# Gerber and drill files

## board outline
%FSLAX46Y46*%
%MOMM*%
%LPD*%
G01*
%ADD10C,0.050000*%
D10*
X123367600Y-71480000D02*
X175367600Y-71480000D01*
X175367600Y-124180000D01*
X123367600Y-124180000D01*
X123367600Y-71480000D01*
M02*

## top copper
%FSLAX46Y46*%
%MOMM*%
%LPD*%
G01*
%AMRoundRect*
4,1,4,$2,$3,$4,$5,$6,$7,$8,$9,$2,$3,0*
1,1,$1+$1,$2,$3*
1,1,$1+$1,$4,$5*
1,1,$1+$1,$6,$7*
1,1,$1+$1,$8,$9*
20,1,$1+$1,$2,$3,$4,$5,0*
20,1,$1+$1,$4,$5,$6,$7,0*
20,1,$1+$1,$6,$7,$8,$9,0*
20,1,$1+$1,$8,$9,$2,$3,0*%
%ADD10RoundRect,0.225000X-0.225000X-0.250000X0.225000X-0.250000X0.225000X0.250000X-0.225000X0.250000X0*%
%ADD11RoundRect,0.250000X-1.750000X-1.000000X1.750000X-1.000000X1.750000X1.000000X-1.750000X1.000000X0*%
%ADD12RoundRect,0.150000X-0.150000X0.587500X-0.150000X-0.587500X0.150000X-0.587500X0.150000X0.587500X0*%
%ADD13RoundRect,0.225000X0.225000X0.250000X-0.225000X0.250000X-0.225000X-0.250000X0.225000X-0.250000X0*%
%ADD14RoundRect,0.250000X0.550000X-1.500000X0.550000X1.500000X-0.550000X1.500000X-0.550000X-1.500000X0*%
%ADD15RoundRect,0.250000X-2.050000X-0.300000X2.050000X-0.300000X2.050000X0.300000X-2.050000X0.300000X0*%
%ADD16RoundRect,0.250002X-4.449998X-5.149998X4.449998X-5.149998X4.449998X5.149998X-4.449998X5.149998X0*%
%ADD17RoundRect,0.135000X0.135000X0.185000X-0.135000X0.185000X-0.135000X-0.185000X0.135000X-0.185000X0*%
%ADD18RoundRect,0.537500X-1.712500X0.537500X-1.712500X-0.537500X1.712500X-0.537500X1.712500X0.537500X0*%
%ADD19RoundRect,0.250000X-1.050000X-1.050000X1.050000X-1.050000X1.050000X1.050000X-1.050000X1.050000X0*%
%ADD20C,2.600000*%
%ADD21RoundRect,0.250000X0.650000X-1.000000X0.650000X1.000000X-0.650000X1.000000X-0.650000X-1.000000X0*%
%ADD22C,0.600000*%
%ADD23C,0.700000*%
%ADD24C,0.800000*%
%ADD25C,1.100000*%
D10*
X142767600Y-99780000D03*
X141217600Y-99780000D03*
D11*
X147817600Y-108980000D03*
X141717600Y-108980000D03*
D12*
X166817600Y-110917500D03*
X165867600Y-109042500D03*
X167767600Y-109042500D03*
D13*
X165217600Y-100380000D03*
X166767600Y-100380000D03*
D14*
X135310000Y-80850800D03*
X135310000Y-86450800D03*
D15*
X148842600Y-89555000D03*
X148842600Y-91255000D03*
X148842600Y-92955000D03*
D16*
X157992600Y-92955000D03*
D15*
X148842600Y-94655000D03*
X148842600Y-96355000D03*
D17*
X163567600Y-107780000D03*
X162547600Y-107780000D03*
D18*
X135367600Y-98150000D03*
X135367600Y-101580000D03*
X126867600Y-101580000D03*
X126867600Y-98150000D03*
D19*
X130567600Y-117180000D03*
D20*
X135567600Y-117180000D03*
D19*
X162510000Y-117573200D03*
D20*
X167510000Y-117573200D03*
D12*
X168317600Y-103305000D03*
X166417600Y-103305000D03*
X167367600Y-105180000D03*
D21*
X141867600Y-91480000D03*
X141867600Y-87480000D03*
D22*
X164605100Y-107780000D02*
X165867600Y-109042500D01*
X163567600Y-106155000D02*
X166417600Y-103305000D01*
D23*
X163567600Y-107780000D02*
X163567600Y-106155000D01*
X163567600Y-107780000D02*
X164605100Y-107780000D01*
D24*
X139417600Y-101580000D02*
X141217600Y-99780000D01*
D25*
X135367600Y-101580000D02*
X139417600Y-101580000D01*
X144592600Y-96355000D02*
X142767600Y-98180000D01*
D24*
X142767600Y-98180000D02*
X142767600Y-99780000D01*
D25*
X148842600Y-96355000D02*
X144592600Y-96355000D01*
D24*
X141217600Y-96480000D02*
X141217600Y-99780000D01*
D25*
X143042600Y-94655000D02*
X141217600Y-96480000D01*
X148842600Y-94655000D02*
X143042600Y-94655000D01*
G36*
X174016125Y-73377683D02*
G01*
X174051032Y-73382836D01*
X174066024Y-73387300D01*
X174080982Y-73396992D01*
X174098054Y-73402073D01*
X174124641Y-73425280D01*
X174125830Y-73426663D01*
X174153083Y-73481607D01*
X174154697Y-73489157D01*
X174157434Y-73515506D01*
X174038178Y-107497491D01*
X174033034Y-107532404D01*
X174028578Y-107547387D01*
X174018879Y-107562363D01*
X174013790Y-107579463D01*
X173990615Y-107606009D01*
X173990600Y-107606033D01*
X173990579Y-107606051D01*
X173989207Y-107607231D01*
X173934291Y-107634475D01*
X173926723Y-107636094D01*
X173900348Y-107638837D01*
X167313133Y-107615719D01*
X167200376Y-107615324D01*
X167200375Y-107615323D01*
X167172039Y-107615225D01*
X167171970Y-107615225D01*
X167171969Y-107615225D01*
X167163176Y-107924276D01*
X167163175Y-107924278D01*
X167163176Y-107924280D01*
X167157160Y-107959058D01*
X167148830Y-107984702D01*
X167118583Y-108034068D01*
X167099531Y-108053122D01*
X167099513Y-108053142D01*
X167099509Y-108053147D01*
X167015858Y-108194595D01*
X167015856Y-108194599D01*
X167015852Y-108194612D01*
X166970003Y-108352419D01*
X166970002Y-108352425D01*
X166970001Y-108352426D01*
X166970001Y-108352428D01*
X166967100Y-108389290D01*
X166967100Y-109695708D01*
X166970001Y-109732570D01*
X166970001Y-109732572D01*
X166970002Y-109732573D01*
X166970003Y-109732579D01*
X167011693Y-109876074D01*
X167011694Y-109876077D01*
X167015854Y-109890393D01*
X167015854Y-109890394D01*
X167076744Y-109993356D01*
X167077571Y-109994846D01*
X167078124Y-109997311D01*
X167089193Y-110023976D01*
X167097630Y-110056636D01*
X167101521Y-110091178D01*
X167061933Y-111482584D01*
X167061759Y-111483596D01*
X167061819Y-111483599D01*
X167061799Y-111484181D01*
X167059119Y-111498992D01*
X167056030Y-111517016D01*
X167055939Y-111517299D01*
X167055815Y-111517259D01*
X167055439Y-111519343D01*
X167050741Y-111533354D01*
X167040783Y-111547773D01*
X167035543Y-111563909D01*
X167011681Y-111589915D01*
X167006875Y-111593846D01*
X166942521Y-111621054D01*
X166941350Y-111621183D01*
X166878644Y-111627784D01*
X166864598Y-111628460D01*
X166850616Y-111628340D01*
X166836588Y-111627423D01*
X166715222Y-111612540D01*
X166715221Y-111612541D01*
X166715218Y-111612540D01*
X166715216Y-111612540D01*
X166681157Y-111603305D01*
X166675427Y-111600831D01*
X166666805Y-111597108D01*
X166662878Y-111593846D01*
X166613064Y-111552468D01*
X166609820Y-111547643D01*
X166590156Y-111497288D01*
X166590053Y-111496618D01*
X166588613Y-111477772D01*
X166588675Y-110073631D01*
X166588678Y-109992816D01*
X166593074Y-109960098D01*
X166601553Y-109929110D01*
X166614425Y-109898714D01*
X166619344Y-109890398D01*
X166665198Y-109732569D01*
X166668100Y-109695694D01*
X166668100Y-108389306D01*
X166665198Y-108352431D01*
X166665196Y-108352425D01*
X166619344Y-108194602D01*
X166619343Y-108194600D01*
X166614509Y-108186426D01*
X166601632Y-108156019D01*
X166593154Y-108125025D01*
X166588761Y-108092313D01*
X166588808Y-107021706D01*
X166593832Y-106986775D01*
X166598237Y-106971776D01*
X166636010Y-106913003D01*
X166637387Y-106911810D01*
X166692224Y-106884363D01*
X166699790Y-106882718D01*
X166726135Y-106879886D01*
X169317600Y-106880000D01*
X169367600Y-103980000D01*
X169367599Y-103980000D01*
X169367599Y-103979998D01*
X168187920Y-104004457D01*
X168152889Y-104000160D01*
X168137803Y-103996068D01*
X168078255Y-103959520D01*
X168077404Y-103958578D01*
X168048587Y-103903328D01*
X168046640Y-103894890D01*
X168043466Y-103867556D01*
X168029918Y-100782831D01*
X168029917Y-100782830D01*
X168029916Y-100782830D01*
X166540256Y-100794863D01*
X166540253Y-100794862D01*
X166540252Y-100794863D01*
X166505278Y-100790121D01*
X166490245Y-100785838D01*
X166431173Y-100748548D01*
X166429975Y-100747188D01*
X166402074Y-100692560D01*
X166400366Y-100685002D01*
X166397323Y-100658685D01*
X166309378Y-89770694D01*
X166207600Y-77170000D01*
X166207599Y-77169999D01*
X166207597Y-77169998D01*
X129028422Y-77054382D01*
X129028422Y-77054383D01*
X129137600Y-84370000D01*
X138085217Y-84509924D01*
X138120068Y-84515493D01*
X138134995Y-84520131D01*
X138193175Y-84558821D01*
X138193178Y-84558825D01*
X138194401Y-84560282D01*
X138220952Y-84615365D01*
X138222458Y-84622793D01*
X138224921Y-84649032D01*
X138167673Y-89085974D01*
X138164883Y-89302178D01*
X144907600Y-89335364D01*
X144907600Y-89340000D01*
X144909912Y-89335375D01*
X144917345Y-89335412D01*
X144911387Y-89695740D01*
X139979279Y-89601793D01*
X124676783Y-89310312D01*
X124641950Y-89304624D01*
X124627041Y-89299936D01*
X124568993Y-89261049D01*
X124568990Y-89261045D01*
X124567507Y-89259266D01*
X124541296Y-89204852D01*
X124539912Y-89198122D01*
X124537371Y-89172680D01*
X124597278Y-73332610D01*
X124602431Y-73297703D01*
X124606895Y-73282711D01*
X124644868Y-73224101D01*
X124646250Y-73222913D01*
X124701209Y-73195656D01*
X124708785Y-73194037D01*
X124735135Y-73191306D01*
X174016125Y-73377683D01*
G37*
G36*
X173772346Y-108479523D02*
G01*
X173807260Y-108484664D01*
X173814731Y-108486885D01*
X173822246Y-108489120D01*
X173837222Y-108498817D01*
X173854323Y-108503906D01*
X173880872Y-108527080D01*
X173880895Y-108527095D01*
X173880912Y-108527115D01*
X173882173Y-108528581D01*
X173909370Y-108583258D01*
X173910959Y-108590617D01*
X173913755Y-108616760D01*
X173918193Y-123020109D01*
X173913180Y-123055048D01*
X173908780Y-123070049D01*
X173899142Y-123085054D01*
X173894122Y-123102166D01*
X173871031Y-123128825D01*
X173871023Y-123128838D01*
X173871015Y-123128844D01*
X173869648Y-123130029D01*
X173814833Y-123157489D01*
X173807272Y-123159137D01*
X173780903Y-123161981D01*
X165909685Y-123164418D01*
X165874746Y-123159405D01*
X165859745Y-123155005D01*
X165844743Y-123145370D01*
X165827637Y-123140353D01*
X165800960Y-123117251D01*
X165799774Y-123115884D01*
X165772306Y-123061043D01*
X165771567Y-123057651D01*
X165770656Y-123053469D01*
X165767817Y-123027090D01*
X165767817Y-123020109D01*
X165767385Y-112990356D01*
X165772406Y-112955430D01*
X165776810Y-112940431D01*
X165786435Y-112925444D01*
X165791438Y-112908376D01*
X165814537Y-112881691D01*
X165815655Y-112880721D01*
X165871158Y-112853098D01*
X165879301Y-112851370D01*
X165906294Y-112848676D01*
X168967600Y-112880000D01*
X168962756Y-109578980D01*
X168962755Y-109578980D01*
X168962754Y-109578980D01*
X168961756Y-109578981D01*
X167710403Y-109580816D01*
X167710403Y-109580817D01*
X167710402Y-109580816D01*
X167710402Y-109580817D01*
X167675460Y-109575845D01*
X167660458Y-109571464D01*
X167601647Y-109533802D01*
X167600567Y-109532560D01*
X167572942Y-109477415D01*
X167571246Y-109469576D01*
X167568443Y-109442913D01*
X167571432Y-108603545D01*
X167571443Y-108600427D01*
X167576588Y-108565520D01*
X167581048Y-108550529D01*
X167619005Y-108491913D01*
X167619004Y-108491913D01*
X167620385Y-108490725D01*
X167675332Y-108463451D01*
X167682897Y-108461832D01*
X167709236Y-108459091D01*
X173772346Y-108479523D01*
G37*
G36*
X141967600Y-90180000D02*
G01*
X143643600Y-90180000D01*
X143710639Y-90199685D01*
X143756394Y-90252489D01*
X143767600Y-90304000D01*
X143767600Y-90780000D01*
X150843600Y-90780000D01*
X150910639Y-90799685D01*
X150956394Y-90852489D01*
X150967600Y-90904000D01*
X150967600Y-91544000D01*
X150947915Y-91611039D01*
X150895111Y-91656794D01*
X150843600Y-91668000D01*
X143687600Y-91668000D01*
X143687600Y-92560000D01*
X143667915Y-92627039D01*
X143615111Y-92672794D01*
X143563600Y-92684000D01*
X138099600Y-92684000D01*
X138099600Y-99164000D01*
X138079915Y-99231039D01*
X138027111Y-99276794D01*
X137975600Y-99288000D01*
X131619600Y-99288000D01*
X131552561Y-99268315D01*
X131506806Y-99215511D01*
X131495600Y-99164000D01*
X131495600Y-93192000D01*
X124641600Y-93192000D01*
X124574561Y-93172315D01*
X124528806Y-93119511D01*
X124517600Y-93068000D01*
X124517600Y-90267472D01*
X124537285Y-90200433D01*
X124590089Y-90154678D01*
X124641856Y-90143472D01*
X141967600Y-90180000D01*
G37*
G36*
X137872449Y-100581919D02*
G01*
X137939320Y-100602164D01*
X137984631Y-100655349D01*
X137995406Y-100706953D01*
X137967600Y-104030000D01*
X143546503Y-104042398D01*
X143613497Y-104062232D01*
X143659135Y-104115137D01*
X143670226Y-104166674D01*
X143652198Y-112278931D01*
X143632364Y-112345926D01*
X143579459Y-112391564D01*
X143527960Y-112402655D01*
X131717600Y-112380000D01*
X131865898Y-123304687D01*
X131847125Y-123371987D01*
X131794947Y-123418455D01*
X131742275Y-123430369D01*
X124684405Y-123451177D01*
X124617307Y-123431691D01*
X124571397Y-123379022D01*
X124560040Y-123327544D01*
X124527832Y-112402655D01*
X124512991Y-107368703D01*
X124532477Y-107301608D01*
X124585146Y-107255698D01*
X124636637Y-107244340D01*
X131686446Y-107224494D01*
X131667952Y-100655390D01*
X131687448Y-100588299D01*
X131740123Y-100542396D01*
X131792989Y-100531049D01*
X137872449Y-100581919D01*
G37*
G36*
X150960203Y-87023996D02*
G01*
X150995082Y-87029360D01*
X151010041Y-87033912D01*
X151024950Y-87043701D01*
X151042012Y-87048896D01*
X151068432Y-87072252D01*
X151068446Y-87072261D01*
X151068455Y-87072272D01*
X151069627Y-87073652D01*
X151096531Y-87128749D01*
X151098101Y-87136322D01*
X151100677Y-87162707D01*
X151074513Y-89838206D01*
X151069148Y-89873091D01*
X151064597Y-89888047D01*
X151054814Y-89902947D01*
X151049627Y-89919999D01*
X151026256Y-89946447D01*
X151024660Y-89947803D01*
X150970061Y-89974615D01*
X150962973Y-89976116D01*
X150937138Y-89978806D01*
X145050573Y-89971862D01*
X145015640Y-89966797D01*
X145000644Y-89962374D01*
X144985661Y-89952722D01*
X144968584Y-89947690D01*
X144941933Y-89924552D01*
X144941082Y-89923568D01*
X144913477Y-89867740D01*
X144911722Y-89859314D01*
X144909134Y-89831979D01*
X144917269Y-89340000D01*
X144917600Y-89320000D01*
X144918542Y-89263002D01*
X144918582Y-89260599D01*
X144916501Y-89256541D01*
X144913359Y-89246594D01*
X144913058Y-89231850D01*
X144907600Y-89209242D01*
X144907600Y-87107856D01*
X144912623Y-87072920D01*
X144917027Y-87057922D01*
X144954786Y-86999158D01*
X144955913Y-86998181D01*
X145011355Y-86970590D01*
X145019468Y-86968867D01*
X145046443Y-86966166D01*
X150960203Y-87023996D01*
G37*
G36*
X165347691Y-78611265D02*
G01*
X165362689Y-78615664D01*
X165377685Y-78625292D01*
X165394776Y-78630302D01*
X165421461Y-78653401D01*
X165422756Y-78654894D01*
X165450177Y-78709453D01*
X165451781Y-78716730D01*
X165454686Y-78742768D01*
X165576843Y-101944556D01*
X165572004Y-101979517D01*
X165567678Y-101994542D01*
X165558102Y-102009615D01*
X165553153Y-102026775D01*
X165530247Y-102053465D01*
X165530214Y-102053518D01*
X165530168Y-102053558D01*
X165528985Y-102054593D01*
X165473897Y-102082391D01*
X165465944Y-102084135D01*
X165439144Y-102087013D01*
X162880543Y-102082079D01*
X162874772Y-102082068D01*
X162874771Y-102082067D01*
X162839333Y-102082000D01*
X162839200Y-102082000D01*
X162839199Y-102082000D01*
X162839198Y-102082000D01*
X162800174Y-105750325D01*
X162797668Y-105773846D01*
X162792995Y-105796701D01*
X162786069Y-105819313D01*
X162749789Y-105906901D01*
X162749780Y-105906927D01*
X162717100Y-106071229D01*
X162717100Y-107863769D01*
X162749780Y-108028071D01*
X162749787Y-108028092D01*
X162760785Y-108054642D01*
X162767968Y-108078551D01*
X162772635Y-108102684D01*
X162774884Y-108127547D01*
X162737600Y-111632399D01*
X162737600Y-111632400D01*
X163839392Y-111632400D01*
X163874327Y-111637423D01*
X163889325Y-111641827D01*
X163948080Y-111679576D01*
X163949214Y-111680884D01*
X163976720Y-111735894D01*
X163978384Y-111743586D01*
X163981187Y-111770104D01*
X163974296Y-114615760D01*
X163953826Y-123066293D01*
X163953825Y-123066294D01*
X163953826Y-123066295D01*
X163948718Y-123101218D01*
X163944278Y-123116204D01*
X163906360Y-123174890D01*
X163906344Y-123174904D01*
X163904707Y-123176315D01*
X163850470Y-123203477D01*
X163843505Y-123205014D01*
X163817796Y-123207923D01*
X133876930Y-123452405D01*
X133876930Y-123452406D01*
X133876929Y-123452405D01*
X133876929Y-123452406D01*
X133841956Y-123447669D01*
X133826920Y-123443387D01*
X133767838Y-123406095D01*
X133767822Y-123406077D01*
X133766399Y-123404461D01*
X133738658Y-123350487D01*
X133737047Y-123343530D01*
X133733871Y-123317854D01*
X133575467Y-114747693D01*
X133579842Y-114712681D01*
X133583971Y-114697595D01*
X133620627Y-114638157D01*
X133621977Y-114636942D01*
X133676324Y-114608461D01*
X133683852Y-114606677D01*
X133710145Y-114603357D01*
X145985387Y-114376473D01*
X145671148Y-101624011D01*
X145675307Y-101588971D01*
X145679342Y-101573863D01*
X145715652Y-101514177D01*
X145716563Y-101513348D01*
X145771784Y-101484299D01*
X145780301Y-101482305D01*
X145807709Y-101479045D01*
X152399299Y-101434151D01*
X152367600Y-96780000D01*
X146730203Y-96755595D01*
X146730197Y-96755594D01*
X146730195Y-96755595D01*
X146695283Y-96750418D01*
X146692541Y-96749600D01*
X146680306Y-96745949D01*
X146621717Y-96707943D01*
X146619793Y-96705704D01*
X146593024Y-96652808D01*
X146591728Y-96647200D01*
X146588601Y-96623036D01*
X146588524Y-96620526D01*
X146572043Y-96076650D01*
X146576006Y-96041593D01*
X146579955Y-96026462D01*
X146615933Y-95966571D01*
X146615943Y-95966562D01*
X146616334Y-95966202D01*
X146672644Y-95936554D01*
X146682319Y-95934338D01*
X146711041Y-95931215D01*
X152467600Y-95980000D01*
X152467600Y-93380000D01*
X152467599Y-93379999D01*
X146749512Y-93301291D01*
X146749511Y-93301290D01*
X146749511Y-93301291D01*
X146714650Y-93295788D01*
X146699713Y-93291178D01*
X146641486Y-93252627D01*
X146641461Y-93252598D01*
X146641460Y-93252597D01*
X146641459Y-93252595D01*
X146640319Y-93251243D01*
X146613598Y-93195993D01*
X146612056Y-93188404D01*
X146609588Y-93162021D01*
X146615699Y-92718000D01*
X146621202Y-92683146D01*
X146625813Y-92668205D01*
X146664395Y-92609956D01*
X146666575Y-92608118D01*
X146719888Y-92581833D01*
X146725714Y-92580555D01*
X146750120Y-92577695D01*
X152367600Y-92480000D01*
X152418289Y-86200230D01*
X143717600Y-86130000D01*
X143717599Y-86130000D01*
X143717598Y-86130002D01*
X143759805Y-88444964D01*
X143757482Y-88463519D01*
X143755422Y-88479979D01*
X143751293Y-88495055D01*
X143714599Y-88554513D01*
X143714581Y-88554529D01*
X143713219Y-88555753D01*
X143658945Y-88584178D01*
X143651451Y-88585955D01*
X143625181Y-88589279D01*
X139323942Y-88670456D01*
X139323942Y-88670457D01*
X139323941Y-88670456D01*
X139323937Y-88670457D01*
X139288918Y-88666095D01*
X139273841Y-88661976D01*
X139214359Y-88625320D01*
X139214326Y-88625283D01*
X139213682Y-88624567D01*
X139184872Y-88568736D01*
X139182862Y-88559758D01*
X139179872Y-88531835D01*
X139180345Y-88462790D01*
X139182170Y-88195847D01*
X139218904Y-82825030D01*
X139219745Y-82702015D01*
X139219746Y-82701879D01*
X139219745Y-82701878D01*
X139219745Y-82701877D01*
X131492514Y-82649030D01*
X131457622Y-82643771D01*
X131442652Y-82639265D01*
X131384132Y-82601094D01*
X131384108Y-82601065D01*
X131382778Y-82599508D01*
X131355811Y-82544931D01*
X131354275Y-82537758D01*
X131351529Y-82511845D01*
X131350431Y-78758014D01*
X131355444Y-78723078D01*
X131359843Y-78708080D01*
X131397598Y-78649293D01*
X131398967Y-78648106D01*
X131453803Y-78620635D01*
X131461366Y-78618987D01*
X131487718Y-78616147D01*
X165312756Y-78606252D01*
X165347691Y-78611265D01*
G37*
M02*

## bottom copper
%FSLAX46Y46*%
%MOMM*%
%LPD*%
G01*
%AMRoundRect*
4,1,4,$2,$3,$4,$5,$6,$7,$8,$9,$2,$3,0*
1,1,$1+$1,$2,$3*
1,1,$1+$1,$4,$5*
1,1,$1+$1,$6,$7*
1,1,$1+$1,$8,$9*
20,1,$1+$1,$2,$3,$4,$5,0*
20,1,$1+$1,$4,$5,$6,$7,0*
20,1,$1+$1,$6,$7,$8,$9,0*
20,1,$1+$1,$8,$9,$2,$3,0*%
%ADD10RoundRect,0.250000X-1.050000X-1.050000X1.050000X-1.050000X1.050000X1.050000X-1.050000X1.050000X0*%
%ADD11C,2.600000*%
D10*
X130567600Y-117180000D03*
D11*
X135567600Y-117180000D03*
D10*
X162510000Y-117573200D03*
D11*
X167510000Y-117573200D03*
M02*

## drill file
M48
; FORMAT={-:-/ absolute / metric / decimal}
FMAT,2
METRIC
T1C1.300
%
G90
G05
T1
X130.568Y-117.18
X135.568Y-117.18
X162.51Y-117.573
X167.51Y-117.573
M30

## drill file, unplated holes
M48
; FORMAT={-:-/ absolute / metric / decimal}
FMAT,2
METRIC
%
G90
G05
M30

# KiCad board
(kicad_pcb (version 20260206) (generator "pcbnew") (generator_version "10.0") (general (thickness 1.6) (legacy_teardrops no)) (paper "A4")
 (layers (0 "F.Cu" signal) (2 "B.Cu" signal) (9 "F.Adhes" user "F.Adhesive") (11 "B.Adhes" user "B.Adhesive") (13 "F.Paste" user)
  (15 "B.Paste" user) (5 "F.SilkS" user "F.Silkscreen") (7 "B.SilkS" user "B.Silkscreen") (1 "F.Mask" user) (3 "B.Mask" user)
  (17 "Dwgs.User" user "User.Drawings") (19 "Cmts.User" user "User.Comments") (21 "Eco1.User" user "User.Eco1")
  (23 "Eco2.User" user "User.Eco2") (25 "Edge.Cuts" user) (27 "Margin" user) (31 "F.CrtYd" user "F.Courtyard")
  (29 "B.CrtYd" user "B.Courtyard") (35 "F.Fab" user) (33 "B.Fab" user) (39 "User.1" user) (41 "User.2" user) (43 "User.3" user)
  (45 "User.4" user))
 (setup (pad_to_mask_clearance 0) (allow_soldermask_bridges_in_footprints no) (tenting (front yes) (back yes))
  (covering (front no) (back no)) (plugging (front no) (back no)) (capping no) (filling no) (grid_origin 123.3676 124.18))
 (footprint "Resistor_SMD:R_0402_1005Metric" (layer "F.Cu") (at 163.0576 107.78 180)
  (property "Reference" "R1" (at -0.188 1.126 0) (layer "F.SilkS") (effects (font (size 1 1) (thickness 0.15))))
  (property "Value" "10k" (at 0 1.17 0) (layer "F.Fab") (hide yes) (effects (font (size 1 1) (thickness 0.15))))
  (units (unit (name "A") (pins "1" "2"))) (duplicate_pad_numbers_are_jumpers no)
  (pad "1" smd roundrect (at -0.51 0 180) (size 0.54 0.64) (layers "F.Cu" "F.Mask" "F.Paste") (roundrect_rratio 0.25) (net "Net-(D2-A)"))
  (pad "2" smd roundrect (at 0.51 0 180) (size 0.54 0.64) (layers "F.Cu" "F.Mask" "F.Paste") (roundrect_rratio 0.25) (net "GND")))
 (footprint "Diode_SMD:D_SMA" (layer "F.Cu") (at 141.8676 89.48 90)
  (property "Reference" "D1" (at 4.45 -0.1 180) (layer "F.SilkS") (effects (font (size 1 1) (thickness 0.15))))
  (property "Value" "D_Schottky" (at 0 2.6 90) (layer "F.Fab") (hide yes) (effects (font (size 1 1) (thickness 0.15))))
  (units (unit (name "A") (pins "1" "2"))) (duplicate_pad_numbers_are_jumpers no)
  (pad "1" smd roundrect (at -2 0 90) (size 2.5 1.8) (layers "F.Cu" "F.Mask" "F.Paste") (roundrect_rratio 0.1388888889) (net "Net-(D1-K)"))
  (pad "2" smd roundrect (at 2 0 90) (size 2.5 1.8) (layers "F.Cu" "F.Mask" "F.Paste") (roundrect_rratio 0.1388888889) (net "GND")))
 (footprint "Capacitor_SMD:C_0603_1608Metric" (layer "F.Cu") (at 141.9926 99.78)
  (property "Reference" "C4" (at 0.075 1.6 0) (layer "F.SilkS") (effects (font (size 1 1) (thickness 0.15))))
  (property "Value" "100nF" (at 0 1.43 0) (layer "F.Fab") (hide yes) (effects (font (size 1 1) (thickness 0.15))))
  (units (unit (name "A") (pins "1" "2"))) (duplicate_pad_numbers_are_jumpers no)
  (pad "1" smd roundrect (at -0.775 0) (size 0.9 0.95) (layers "F.Cu" "F.Mask" "F.Paste") (roundrect_rratio 0.25) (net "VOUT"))
  (pad "2" smd roundrect (at 0.775 0) (size 0.9 0.95) (layers "F.Cu" "F.Mask" "F.Paste") (roundrect_rratio 0.25) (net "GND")))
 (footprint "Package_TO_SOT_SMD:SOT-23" (layer "F.Cu") (at 167.3676 104.2425 -90)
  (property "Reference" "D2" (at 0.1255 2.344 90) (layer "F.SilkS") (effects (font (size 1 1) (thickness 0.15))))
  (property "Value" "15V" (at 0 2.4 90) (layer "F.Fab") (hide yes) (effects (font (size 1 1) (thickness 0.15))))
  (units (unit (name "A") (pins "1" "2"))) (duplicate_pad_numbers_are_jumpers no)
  (pad "1" smd roundrect (at -0.9375 -0.95 270) (size 1.475 0.6) (layers "F.Cu" "F.Mask" "F.Paste") (roundrect_rratio 0.25)
   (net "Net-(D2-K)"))
  (pad "2" smd roundrect (at -0.9375 0.95 270) (size 1.475 0.6) (layers "F.Cu" "F.Mask" "F.Paste") (roundrect_rratio 0.25)
   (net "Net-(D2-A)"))
  (pad "3" smd roundrect (at 0.9375 0 270) (size 1.475 0.6) (layers "F.Cu" "F.Mask" "F.Paste") (roundrect_rratio 0.25)))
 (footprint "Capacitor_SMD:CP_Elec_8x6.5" (layer "F.Cu") (at 144.7676 108.98)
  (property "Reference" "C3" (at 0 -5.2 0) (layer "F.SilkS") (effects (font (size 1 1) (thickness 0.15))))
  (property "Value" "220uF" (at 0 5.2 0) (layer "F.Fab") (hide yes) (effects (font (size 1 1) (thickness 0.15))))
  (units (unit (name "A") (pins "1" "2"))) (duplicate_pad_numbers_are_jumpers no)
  (pad "1" smd roundrect (at -3.05 0) (size 4 2.5) (layers "F.Cu" "F.Mask" "F.Paste") (roundrect_rratio 0.1) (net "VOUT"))
  (pad "2" smd roundrect (at 3.05 0) (size 4 2.5) (layers "F.Cu" "F.Mask" "F.Paste") (roundrect_rratio 0.1) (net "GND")))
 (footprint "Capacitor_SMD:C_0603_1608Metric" (layer "F.Cu") (at 165.9926 100.38 180)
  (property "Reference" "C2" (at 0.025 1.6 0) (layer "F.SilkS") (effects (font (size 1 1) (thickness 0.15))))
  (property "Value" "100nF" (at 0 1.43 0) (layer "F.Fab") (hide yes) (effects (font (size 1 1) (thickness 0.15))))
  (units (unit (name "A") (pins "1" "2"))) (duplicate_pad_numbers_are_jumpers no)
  (pad "1" smd roundrect (at -0.775 0 180) (size 0.9 0.95) (layers "F.Cu" "F.Mask" "F.Paste") (roundrect_rratio 0.25) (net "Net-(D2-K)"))
  (pad "2" smd roundrect (at 0.775 0 180) (size 0.9 0.95) (layers "F.Cu" "F.Mask" "F.Paste") (roundrect_rratio 0.25) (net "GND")))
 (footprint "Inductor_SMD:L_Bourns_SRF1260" (layer "F.Cu") (at 131.1176 99.865 -90)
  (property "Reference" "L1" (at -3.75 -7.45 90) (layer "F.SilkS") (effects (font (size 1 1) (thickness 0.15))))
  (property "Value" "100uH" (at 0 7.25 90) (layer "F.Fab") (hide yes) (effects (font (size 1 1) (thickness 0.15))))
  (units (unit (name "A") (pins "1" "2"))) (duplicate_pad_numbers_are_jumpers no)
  (pad "1" smd roundrect (at -1.715 -4.25 270) (size 2.15 4.5) (layers "F.Cu" "F.Mask" "F.Paste") (roundrect_rratio 0.25) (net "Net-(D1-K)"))
  (pad "2" smd roundrect (at 1.715 -4.25 270) (size 2.15 4.5) (layers "F.Cu" "F.Mask" "F.Paste") (roundrect_rratio 0.25) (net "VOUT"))
  (pad "3" smd roundrect (at 1.715 4.25 270) (size 2.15 4.5) (layers "F.Cu" "F.Mask" "F.Paste") (roundrect_rratio 0.25))
  (pad "4" smd roundrect (at -1.715 4.25 270) (size 2.15 4.5) (layers "F.Cu" "F.Mask" "F.Paste") (roundrect_rratio 0.25)))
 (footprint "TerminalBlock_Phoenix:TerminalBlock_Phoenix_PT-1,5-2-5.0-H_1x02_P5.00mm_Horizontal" (layer "F.Cu") (at 130.5676 117.18)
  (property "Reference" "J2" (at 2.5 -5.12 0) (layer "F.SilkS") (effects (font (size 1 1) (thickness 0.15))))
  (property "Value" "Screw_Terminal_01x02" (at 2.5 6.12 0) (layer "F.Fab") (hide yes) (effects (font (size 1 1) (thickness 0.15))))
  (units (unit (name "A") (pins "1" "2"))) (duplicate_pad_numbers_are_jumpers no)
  (pad "1" thru_hole roundrect (at 0 0) (size 2.6 2.6) (drill 1.3) (layers "*.Cu" "*.Mask") (remove_unused_layers no)
   (roundrect_rratio 0.096154) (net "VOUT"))
  (pad "2" thru_hole circle (at 5 0) (size 2.6 2.6) (drill 1.3) (layers "*.Cu" "*.Mask") (remove_unused_layers no) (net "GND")))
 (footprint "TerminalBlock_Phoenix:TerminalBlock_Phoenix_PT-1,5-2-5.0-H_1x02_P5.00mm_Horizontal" (layer "F.Cu") (at 162.51 117.5732)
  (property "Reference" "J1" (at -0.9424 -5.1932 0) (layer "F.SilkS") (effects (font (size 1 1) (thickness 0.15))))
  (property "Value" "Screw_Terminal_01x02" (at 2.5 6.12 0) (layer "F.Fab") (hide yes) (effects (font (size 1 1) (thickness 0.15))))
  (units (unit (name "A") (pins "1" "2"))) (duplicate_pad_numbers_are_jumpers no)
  (pad "1" thru_hole roundrect (at 0 0) (size 2.6 2.6) (drill 1.3) (layers "*.Cu" "*.Mask") (remove_unused_layers no)
   (roundrect_rratio 0.096154) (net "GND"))
  (pad "2" thru_hole circle (at 5 0) (size 2.6 2.6) (drill 1.3) (layers "*.Cu" "*.Mask") (remove_unused_layers no) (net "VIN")))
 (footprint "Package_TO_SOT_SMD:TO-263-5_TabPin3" (layer "F.Cu") (at 156.4926 92.955)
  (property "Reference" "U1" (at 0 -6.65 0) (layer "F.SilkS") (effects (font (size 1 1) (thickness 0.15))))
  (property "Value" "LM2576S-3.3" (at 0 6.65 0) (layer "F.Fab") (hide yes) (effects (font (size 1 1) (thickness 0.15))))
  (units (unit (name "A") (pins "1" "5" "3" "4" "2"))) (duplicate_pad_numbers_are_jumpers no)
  (pad "" smd roundrect (at -0.925 -2.775) (size 4.55 5.25) (layers "F.Paste") (roundrect_rratio 0.054945))
  (pad "" smd roundrect (at -0.925 2.775) (size 4.55 5.25) (layers "F.Paste") (roundrect_rratio 0.054945))
  (pad "" smd roundrect (at 3.925 -2.775) (size 4.55 5.25) (layers "F.Paste") (roundrect_rratio 0.054945))
  (pad "" smd roundrect (at 3.925 2.775) (size 4.55 5.25) (layers "F.Paste") (roundrect_rratio 0.054945))
  (pad "1" smd roundrect (at -7.65 -3.4) (size 4.6 1.1) (layers "F.Cu" "F.Mask" "F.Paste") (roundrect_rratio 0.227273) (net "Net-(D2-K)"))
  (pad "2" smd roundrect (at -7.65 -1.7) (size 4.6 1.1) (layers "F.Cu" "F.Mask" "F.Paste") (roundrect_rratio 0.227273) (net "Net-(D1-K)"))
  (pad "3" smd roundrect (at -7.65 0) (size 4.6 1.1) (layers "F.Cu" "F.Mask" "F.Paste") (roundrect_rratio 0.227273) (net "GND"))
  (pad "3" smd roundrect (at 1.5 0) (size 9.4 10.8) (layers "F.Cu" "F.Mask") (roundrect_rratio 0.026596) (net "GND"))
  (pad "4" smd roundrect (at -7.65 1.7) (size 4.6 1.1) (layers "F.Cu" "F.Mask" "F.Paste") (roundrect_rratio 0.227273) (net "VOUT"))
  (pad "5" smd roundrect (at -7.65 3.4) (size 4.6 1.1) (layers "F.Cu" "F.Mask" "F.Paste") (roundrect_rratio 0.227273) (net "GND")))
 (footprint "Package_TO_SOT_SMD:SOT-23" (layer "F.Cu") (at 166.8176 109.98 -90)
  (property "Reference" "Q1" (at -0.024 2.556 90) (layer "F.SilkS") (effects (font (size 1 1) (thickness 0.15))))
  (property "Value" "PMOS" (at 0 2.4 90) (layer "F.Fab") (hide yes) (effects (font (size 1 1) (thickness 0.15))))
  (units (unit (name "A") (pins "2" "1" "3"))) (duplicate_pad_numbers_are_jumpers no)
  (pad "1" smd roundrect (at -0.9375 -0.95 270) (size 1.475 0.6) (layers "F.Cu" "F.Mask" "F.Paste") (roundrect_rratio 0.25) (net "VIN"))
  (pad "2" smd roundrect (at -0.9375 0.95 270) (size 1.475 0.6) (layers "F.Cu" "F.Mask" "F.Paste") (roundrect_rratio 0.25)
   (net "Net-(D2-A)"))
  (pad "3" smd roundrect (at 0.9375 0 270) (size 1.475 0.6) (layers "F.Cu" "F.Mask" "F.Paste") (roundrect_rratio 0.25) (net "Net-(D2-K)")))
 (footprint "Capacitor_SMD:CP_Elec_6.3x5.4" (layer "F.Cu") (at 135.31 83.6508 90)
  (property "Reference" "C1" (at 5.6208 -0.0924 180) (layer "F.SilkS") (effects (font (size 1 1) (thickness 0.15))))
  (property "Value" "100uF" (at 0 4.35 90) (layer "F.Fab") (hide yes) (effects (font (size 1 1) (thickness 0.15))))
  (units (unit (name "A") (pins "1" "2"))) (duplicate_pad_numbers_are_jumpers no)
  (pad "1" smd roundrect (at -2.8 0 90) (size 3.5 1.6) (layers "F.Cu" "F.Mask" "F.Paste") (roundrect_rratio 0.15625) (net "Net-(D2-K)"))
  (pad "2" smd roundrect (at 2.8 0 90) (size 3.5 1.6) (layers "F.Cu" "F.Mask" "F.Paste") (roundrect_rratio 0.15625) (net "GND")))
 (gr_rect (start 123.3676 71.48) (end 175.3676 124.18) (stroke (width 0.05) (type default)) (fill no) (layer "Edge.Cuts"))
 (segment (start 139.4176 101.58) (end 141.2176 99.78) (width 0.8) (layer "F.Cu") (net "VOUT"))
 (segment (start 148.8426 94.655) (end 143.0426 94.655) (width 1.1) (layer "F.Cu") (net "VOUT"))
 (segment (start 143.0426 94.655) (end 141.2176 96.48) (width 1.1) (layer "F.Cu") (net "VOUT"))
 (segment (start 141.2176 96.48) (end 141.2176 99.78) (width 0.8) (layer "F.Cu") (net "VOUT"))
 (segment (start 135.3676 101.58) (end 139.4176 101.58) (width 1.1) (layer "F.Cu") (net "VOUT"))
 (segment (start 148.8426 96.355) (end 144.5926 96.355) (width 1.1) (layer "F.Cu") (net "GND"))
 (segment (start 144.5926 96.355) (end 142.7676 98.18) (width 1.1) (layer "F.Cu") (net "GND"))
 (segment (start 142.7676 98.18) (end 142.7676 99.78) (width 0.8) (layer "F.Cu") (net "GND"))
 (segment (start 163.5676 107.78) (end 164.6051 107.78) (width 0.7) (layer "F.Cu") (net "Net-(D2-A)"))
 (segment (start 164.6051 107.78) (end 165.8676 109.0425) (width 0.6) (layer "F.Cu") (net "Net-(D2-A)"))
 (segment (start 163.5676 107.78) (end 163.5676 106.155) (width 0.7) (layer "F.Cu") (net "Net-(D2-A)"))
 (segment (start 163.5676 106.155) (end 166.4176 103.305) (width 0.6) (layer "F.Cu") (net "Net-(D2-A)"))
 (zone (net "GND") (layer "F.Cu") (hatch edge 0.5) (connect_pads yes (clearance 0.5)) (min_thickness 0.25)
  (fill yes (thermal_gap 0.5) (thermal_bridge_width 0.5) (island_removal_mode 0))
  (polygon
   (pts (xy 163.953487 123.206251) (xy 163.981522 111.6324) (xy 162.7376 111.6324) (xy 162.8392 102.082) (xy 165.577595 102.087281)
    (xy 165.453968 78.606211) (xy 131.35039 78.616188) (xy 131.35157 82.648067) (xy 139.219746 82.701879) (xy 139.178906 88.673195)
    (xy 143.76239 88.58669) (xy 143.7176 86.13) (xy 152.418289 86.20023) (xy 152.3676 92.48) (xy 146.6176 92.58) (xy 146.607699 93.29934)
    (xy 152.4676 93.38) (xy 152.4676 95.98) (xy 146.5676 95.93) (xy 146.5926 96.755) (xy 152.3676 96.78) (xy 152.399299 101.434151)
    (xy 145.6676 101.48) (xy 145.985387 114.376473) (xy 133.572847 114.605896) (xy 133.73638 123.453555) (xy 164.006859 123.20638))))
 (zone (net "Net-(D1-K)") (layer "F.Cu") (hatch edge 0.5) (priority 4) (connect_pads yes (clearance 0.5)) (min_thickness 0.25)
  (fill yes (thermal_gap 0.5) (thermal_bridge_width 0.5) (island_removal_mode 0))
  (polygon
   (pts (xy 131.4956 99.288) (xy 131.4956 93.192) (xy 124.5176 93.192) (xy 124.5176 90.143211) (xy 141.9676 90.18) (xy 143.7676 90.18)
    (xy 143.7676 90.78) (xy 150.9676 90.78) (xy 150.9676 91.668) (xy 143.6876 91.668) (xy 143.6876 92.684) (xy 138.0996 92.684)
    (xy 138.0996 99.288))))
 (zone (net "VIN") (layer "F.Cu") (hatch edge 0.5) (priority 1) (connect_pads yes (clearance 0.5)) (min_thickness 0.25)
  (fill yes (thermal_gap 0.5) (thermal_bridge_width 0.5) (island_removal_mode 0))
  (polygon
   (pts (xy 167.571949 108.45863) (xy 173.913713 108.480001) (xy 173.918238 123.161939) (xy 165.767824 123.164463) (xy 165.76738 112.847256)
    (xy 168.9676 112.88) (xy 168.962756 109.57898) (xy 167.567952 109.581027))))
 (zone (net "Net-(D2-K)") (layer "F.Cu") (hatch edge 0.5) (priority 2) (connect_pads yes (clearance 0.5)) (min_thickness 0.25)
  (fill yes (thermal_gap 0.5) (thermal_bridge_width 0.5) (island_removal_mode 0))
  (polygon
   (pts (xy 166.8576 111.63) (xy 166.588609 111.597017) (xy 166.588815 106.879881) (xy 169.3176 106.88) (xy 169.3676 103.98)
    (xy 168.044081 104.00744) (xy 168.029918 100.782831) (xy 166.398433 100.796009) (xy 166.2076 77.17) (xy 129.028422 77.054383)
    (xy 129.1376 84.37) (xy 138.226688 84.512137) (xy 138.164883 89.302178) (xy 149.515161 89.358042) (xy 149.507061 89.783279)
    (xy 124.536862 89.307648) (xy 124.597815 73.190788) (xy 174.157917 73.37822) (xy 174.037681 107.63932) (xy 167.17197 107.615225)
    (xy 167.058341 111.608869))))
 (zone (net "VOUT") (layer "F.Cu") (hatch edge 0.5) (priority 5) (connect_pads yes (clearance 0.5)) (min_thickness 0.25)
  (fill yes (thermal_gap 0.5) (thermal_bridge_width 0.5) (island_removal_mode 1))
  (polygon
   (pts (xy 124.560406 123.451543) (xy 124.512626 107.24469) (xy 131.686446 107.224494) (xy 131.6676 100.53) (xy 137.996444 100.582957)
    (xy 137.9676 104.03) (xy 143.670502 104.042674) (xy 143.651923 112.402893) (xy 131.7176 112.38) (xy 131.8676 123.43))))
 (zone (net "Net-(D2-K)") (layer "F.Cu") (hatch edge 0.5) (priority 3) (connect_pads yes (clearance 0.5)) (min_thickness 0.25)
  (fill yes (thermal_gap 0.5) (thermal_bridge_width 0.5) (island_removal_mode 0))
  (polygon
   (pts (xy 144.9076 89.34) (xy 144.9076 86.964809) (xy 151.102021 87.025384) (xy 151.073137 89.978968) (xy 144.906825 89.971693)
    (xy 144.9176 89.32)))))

